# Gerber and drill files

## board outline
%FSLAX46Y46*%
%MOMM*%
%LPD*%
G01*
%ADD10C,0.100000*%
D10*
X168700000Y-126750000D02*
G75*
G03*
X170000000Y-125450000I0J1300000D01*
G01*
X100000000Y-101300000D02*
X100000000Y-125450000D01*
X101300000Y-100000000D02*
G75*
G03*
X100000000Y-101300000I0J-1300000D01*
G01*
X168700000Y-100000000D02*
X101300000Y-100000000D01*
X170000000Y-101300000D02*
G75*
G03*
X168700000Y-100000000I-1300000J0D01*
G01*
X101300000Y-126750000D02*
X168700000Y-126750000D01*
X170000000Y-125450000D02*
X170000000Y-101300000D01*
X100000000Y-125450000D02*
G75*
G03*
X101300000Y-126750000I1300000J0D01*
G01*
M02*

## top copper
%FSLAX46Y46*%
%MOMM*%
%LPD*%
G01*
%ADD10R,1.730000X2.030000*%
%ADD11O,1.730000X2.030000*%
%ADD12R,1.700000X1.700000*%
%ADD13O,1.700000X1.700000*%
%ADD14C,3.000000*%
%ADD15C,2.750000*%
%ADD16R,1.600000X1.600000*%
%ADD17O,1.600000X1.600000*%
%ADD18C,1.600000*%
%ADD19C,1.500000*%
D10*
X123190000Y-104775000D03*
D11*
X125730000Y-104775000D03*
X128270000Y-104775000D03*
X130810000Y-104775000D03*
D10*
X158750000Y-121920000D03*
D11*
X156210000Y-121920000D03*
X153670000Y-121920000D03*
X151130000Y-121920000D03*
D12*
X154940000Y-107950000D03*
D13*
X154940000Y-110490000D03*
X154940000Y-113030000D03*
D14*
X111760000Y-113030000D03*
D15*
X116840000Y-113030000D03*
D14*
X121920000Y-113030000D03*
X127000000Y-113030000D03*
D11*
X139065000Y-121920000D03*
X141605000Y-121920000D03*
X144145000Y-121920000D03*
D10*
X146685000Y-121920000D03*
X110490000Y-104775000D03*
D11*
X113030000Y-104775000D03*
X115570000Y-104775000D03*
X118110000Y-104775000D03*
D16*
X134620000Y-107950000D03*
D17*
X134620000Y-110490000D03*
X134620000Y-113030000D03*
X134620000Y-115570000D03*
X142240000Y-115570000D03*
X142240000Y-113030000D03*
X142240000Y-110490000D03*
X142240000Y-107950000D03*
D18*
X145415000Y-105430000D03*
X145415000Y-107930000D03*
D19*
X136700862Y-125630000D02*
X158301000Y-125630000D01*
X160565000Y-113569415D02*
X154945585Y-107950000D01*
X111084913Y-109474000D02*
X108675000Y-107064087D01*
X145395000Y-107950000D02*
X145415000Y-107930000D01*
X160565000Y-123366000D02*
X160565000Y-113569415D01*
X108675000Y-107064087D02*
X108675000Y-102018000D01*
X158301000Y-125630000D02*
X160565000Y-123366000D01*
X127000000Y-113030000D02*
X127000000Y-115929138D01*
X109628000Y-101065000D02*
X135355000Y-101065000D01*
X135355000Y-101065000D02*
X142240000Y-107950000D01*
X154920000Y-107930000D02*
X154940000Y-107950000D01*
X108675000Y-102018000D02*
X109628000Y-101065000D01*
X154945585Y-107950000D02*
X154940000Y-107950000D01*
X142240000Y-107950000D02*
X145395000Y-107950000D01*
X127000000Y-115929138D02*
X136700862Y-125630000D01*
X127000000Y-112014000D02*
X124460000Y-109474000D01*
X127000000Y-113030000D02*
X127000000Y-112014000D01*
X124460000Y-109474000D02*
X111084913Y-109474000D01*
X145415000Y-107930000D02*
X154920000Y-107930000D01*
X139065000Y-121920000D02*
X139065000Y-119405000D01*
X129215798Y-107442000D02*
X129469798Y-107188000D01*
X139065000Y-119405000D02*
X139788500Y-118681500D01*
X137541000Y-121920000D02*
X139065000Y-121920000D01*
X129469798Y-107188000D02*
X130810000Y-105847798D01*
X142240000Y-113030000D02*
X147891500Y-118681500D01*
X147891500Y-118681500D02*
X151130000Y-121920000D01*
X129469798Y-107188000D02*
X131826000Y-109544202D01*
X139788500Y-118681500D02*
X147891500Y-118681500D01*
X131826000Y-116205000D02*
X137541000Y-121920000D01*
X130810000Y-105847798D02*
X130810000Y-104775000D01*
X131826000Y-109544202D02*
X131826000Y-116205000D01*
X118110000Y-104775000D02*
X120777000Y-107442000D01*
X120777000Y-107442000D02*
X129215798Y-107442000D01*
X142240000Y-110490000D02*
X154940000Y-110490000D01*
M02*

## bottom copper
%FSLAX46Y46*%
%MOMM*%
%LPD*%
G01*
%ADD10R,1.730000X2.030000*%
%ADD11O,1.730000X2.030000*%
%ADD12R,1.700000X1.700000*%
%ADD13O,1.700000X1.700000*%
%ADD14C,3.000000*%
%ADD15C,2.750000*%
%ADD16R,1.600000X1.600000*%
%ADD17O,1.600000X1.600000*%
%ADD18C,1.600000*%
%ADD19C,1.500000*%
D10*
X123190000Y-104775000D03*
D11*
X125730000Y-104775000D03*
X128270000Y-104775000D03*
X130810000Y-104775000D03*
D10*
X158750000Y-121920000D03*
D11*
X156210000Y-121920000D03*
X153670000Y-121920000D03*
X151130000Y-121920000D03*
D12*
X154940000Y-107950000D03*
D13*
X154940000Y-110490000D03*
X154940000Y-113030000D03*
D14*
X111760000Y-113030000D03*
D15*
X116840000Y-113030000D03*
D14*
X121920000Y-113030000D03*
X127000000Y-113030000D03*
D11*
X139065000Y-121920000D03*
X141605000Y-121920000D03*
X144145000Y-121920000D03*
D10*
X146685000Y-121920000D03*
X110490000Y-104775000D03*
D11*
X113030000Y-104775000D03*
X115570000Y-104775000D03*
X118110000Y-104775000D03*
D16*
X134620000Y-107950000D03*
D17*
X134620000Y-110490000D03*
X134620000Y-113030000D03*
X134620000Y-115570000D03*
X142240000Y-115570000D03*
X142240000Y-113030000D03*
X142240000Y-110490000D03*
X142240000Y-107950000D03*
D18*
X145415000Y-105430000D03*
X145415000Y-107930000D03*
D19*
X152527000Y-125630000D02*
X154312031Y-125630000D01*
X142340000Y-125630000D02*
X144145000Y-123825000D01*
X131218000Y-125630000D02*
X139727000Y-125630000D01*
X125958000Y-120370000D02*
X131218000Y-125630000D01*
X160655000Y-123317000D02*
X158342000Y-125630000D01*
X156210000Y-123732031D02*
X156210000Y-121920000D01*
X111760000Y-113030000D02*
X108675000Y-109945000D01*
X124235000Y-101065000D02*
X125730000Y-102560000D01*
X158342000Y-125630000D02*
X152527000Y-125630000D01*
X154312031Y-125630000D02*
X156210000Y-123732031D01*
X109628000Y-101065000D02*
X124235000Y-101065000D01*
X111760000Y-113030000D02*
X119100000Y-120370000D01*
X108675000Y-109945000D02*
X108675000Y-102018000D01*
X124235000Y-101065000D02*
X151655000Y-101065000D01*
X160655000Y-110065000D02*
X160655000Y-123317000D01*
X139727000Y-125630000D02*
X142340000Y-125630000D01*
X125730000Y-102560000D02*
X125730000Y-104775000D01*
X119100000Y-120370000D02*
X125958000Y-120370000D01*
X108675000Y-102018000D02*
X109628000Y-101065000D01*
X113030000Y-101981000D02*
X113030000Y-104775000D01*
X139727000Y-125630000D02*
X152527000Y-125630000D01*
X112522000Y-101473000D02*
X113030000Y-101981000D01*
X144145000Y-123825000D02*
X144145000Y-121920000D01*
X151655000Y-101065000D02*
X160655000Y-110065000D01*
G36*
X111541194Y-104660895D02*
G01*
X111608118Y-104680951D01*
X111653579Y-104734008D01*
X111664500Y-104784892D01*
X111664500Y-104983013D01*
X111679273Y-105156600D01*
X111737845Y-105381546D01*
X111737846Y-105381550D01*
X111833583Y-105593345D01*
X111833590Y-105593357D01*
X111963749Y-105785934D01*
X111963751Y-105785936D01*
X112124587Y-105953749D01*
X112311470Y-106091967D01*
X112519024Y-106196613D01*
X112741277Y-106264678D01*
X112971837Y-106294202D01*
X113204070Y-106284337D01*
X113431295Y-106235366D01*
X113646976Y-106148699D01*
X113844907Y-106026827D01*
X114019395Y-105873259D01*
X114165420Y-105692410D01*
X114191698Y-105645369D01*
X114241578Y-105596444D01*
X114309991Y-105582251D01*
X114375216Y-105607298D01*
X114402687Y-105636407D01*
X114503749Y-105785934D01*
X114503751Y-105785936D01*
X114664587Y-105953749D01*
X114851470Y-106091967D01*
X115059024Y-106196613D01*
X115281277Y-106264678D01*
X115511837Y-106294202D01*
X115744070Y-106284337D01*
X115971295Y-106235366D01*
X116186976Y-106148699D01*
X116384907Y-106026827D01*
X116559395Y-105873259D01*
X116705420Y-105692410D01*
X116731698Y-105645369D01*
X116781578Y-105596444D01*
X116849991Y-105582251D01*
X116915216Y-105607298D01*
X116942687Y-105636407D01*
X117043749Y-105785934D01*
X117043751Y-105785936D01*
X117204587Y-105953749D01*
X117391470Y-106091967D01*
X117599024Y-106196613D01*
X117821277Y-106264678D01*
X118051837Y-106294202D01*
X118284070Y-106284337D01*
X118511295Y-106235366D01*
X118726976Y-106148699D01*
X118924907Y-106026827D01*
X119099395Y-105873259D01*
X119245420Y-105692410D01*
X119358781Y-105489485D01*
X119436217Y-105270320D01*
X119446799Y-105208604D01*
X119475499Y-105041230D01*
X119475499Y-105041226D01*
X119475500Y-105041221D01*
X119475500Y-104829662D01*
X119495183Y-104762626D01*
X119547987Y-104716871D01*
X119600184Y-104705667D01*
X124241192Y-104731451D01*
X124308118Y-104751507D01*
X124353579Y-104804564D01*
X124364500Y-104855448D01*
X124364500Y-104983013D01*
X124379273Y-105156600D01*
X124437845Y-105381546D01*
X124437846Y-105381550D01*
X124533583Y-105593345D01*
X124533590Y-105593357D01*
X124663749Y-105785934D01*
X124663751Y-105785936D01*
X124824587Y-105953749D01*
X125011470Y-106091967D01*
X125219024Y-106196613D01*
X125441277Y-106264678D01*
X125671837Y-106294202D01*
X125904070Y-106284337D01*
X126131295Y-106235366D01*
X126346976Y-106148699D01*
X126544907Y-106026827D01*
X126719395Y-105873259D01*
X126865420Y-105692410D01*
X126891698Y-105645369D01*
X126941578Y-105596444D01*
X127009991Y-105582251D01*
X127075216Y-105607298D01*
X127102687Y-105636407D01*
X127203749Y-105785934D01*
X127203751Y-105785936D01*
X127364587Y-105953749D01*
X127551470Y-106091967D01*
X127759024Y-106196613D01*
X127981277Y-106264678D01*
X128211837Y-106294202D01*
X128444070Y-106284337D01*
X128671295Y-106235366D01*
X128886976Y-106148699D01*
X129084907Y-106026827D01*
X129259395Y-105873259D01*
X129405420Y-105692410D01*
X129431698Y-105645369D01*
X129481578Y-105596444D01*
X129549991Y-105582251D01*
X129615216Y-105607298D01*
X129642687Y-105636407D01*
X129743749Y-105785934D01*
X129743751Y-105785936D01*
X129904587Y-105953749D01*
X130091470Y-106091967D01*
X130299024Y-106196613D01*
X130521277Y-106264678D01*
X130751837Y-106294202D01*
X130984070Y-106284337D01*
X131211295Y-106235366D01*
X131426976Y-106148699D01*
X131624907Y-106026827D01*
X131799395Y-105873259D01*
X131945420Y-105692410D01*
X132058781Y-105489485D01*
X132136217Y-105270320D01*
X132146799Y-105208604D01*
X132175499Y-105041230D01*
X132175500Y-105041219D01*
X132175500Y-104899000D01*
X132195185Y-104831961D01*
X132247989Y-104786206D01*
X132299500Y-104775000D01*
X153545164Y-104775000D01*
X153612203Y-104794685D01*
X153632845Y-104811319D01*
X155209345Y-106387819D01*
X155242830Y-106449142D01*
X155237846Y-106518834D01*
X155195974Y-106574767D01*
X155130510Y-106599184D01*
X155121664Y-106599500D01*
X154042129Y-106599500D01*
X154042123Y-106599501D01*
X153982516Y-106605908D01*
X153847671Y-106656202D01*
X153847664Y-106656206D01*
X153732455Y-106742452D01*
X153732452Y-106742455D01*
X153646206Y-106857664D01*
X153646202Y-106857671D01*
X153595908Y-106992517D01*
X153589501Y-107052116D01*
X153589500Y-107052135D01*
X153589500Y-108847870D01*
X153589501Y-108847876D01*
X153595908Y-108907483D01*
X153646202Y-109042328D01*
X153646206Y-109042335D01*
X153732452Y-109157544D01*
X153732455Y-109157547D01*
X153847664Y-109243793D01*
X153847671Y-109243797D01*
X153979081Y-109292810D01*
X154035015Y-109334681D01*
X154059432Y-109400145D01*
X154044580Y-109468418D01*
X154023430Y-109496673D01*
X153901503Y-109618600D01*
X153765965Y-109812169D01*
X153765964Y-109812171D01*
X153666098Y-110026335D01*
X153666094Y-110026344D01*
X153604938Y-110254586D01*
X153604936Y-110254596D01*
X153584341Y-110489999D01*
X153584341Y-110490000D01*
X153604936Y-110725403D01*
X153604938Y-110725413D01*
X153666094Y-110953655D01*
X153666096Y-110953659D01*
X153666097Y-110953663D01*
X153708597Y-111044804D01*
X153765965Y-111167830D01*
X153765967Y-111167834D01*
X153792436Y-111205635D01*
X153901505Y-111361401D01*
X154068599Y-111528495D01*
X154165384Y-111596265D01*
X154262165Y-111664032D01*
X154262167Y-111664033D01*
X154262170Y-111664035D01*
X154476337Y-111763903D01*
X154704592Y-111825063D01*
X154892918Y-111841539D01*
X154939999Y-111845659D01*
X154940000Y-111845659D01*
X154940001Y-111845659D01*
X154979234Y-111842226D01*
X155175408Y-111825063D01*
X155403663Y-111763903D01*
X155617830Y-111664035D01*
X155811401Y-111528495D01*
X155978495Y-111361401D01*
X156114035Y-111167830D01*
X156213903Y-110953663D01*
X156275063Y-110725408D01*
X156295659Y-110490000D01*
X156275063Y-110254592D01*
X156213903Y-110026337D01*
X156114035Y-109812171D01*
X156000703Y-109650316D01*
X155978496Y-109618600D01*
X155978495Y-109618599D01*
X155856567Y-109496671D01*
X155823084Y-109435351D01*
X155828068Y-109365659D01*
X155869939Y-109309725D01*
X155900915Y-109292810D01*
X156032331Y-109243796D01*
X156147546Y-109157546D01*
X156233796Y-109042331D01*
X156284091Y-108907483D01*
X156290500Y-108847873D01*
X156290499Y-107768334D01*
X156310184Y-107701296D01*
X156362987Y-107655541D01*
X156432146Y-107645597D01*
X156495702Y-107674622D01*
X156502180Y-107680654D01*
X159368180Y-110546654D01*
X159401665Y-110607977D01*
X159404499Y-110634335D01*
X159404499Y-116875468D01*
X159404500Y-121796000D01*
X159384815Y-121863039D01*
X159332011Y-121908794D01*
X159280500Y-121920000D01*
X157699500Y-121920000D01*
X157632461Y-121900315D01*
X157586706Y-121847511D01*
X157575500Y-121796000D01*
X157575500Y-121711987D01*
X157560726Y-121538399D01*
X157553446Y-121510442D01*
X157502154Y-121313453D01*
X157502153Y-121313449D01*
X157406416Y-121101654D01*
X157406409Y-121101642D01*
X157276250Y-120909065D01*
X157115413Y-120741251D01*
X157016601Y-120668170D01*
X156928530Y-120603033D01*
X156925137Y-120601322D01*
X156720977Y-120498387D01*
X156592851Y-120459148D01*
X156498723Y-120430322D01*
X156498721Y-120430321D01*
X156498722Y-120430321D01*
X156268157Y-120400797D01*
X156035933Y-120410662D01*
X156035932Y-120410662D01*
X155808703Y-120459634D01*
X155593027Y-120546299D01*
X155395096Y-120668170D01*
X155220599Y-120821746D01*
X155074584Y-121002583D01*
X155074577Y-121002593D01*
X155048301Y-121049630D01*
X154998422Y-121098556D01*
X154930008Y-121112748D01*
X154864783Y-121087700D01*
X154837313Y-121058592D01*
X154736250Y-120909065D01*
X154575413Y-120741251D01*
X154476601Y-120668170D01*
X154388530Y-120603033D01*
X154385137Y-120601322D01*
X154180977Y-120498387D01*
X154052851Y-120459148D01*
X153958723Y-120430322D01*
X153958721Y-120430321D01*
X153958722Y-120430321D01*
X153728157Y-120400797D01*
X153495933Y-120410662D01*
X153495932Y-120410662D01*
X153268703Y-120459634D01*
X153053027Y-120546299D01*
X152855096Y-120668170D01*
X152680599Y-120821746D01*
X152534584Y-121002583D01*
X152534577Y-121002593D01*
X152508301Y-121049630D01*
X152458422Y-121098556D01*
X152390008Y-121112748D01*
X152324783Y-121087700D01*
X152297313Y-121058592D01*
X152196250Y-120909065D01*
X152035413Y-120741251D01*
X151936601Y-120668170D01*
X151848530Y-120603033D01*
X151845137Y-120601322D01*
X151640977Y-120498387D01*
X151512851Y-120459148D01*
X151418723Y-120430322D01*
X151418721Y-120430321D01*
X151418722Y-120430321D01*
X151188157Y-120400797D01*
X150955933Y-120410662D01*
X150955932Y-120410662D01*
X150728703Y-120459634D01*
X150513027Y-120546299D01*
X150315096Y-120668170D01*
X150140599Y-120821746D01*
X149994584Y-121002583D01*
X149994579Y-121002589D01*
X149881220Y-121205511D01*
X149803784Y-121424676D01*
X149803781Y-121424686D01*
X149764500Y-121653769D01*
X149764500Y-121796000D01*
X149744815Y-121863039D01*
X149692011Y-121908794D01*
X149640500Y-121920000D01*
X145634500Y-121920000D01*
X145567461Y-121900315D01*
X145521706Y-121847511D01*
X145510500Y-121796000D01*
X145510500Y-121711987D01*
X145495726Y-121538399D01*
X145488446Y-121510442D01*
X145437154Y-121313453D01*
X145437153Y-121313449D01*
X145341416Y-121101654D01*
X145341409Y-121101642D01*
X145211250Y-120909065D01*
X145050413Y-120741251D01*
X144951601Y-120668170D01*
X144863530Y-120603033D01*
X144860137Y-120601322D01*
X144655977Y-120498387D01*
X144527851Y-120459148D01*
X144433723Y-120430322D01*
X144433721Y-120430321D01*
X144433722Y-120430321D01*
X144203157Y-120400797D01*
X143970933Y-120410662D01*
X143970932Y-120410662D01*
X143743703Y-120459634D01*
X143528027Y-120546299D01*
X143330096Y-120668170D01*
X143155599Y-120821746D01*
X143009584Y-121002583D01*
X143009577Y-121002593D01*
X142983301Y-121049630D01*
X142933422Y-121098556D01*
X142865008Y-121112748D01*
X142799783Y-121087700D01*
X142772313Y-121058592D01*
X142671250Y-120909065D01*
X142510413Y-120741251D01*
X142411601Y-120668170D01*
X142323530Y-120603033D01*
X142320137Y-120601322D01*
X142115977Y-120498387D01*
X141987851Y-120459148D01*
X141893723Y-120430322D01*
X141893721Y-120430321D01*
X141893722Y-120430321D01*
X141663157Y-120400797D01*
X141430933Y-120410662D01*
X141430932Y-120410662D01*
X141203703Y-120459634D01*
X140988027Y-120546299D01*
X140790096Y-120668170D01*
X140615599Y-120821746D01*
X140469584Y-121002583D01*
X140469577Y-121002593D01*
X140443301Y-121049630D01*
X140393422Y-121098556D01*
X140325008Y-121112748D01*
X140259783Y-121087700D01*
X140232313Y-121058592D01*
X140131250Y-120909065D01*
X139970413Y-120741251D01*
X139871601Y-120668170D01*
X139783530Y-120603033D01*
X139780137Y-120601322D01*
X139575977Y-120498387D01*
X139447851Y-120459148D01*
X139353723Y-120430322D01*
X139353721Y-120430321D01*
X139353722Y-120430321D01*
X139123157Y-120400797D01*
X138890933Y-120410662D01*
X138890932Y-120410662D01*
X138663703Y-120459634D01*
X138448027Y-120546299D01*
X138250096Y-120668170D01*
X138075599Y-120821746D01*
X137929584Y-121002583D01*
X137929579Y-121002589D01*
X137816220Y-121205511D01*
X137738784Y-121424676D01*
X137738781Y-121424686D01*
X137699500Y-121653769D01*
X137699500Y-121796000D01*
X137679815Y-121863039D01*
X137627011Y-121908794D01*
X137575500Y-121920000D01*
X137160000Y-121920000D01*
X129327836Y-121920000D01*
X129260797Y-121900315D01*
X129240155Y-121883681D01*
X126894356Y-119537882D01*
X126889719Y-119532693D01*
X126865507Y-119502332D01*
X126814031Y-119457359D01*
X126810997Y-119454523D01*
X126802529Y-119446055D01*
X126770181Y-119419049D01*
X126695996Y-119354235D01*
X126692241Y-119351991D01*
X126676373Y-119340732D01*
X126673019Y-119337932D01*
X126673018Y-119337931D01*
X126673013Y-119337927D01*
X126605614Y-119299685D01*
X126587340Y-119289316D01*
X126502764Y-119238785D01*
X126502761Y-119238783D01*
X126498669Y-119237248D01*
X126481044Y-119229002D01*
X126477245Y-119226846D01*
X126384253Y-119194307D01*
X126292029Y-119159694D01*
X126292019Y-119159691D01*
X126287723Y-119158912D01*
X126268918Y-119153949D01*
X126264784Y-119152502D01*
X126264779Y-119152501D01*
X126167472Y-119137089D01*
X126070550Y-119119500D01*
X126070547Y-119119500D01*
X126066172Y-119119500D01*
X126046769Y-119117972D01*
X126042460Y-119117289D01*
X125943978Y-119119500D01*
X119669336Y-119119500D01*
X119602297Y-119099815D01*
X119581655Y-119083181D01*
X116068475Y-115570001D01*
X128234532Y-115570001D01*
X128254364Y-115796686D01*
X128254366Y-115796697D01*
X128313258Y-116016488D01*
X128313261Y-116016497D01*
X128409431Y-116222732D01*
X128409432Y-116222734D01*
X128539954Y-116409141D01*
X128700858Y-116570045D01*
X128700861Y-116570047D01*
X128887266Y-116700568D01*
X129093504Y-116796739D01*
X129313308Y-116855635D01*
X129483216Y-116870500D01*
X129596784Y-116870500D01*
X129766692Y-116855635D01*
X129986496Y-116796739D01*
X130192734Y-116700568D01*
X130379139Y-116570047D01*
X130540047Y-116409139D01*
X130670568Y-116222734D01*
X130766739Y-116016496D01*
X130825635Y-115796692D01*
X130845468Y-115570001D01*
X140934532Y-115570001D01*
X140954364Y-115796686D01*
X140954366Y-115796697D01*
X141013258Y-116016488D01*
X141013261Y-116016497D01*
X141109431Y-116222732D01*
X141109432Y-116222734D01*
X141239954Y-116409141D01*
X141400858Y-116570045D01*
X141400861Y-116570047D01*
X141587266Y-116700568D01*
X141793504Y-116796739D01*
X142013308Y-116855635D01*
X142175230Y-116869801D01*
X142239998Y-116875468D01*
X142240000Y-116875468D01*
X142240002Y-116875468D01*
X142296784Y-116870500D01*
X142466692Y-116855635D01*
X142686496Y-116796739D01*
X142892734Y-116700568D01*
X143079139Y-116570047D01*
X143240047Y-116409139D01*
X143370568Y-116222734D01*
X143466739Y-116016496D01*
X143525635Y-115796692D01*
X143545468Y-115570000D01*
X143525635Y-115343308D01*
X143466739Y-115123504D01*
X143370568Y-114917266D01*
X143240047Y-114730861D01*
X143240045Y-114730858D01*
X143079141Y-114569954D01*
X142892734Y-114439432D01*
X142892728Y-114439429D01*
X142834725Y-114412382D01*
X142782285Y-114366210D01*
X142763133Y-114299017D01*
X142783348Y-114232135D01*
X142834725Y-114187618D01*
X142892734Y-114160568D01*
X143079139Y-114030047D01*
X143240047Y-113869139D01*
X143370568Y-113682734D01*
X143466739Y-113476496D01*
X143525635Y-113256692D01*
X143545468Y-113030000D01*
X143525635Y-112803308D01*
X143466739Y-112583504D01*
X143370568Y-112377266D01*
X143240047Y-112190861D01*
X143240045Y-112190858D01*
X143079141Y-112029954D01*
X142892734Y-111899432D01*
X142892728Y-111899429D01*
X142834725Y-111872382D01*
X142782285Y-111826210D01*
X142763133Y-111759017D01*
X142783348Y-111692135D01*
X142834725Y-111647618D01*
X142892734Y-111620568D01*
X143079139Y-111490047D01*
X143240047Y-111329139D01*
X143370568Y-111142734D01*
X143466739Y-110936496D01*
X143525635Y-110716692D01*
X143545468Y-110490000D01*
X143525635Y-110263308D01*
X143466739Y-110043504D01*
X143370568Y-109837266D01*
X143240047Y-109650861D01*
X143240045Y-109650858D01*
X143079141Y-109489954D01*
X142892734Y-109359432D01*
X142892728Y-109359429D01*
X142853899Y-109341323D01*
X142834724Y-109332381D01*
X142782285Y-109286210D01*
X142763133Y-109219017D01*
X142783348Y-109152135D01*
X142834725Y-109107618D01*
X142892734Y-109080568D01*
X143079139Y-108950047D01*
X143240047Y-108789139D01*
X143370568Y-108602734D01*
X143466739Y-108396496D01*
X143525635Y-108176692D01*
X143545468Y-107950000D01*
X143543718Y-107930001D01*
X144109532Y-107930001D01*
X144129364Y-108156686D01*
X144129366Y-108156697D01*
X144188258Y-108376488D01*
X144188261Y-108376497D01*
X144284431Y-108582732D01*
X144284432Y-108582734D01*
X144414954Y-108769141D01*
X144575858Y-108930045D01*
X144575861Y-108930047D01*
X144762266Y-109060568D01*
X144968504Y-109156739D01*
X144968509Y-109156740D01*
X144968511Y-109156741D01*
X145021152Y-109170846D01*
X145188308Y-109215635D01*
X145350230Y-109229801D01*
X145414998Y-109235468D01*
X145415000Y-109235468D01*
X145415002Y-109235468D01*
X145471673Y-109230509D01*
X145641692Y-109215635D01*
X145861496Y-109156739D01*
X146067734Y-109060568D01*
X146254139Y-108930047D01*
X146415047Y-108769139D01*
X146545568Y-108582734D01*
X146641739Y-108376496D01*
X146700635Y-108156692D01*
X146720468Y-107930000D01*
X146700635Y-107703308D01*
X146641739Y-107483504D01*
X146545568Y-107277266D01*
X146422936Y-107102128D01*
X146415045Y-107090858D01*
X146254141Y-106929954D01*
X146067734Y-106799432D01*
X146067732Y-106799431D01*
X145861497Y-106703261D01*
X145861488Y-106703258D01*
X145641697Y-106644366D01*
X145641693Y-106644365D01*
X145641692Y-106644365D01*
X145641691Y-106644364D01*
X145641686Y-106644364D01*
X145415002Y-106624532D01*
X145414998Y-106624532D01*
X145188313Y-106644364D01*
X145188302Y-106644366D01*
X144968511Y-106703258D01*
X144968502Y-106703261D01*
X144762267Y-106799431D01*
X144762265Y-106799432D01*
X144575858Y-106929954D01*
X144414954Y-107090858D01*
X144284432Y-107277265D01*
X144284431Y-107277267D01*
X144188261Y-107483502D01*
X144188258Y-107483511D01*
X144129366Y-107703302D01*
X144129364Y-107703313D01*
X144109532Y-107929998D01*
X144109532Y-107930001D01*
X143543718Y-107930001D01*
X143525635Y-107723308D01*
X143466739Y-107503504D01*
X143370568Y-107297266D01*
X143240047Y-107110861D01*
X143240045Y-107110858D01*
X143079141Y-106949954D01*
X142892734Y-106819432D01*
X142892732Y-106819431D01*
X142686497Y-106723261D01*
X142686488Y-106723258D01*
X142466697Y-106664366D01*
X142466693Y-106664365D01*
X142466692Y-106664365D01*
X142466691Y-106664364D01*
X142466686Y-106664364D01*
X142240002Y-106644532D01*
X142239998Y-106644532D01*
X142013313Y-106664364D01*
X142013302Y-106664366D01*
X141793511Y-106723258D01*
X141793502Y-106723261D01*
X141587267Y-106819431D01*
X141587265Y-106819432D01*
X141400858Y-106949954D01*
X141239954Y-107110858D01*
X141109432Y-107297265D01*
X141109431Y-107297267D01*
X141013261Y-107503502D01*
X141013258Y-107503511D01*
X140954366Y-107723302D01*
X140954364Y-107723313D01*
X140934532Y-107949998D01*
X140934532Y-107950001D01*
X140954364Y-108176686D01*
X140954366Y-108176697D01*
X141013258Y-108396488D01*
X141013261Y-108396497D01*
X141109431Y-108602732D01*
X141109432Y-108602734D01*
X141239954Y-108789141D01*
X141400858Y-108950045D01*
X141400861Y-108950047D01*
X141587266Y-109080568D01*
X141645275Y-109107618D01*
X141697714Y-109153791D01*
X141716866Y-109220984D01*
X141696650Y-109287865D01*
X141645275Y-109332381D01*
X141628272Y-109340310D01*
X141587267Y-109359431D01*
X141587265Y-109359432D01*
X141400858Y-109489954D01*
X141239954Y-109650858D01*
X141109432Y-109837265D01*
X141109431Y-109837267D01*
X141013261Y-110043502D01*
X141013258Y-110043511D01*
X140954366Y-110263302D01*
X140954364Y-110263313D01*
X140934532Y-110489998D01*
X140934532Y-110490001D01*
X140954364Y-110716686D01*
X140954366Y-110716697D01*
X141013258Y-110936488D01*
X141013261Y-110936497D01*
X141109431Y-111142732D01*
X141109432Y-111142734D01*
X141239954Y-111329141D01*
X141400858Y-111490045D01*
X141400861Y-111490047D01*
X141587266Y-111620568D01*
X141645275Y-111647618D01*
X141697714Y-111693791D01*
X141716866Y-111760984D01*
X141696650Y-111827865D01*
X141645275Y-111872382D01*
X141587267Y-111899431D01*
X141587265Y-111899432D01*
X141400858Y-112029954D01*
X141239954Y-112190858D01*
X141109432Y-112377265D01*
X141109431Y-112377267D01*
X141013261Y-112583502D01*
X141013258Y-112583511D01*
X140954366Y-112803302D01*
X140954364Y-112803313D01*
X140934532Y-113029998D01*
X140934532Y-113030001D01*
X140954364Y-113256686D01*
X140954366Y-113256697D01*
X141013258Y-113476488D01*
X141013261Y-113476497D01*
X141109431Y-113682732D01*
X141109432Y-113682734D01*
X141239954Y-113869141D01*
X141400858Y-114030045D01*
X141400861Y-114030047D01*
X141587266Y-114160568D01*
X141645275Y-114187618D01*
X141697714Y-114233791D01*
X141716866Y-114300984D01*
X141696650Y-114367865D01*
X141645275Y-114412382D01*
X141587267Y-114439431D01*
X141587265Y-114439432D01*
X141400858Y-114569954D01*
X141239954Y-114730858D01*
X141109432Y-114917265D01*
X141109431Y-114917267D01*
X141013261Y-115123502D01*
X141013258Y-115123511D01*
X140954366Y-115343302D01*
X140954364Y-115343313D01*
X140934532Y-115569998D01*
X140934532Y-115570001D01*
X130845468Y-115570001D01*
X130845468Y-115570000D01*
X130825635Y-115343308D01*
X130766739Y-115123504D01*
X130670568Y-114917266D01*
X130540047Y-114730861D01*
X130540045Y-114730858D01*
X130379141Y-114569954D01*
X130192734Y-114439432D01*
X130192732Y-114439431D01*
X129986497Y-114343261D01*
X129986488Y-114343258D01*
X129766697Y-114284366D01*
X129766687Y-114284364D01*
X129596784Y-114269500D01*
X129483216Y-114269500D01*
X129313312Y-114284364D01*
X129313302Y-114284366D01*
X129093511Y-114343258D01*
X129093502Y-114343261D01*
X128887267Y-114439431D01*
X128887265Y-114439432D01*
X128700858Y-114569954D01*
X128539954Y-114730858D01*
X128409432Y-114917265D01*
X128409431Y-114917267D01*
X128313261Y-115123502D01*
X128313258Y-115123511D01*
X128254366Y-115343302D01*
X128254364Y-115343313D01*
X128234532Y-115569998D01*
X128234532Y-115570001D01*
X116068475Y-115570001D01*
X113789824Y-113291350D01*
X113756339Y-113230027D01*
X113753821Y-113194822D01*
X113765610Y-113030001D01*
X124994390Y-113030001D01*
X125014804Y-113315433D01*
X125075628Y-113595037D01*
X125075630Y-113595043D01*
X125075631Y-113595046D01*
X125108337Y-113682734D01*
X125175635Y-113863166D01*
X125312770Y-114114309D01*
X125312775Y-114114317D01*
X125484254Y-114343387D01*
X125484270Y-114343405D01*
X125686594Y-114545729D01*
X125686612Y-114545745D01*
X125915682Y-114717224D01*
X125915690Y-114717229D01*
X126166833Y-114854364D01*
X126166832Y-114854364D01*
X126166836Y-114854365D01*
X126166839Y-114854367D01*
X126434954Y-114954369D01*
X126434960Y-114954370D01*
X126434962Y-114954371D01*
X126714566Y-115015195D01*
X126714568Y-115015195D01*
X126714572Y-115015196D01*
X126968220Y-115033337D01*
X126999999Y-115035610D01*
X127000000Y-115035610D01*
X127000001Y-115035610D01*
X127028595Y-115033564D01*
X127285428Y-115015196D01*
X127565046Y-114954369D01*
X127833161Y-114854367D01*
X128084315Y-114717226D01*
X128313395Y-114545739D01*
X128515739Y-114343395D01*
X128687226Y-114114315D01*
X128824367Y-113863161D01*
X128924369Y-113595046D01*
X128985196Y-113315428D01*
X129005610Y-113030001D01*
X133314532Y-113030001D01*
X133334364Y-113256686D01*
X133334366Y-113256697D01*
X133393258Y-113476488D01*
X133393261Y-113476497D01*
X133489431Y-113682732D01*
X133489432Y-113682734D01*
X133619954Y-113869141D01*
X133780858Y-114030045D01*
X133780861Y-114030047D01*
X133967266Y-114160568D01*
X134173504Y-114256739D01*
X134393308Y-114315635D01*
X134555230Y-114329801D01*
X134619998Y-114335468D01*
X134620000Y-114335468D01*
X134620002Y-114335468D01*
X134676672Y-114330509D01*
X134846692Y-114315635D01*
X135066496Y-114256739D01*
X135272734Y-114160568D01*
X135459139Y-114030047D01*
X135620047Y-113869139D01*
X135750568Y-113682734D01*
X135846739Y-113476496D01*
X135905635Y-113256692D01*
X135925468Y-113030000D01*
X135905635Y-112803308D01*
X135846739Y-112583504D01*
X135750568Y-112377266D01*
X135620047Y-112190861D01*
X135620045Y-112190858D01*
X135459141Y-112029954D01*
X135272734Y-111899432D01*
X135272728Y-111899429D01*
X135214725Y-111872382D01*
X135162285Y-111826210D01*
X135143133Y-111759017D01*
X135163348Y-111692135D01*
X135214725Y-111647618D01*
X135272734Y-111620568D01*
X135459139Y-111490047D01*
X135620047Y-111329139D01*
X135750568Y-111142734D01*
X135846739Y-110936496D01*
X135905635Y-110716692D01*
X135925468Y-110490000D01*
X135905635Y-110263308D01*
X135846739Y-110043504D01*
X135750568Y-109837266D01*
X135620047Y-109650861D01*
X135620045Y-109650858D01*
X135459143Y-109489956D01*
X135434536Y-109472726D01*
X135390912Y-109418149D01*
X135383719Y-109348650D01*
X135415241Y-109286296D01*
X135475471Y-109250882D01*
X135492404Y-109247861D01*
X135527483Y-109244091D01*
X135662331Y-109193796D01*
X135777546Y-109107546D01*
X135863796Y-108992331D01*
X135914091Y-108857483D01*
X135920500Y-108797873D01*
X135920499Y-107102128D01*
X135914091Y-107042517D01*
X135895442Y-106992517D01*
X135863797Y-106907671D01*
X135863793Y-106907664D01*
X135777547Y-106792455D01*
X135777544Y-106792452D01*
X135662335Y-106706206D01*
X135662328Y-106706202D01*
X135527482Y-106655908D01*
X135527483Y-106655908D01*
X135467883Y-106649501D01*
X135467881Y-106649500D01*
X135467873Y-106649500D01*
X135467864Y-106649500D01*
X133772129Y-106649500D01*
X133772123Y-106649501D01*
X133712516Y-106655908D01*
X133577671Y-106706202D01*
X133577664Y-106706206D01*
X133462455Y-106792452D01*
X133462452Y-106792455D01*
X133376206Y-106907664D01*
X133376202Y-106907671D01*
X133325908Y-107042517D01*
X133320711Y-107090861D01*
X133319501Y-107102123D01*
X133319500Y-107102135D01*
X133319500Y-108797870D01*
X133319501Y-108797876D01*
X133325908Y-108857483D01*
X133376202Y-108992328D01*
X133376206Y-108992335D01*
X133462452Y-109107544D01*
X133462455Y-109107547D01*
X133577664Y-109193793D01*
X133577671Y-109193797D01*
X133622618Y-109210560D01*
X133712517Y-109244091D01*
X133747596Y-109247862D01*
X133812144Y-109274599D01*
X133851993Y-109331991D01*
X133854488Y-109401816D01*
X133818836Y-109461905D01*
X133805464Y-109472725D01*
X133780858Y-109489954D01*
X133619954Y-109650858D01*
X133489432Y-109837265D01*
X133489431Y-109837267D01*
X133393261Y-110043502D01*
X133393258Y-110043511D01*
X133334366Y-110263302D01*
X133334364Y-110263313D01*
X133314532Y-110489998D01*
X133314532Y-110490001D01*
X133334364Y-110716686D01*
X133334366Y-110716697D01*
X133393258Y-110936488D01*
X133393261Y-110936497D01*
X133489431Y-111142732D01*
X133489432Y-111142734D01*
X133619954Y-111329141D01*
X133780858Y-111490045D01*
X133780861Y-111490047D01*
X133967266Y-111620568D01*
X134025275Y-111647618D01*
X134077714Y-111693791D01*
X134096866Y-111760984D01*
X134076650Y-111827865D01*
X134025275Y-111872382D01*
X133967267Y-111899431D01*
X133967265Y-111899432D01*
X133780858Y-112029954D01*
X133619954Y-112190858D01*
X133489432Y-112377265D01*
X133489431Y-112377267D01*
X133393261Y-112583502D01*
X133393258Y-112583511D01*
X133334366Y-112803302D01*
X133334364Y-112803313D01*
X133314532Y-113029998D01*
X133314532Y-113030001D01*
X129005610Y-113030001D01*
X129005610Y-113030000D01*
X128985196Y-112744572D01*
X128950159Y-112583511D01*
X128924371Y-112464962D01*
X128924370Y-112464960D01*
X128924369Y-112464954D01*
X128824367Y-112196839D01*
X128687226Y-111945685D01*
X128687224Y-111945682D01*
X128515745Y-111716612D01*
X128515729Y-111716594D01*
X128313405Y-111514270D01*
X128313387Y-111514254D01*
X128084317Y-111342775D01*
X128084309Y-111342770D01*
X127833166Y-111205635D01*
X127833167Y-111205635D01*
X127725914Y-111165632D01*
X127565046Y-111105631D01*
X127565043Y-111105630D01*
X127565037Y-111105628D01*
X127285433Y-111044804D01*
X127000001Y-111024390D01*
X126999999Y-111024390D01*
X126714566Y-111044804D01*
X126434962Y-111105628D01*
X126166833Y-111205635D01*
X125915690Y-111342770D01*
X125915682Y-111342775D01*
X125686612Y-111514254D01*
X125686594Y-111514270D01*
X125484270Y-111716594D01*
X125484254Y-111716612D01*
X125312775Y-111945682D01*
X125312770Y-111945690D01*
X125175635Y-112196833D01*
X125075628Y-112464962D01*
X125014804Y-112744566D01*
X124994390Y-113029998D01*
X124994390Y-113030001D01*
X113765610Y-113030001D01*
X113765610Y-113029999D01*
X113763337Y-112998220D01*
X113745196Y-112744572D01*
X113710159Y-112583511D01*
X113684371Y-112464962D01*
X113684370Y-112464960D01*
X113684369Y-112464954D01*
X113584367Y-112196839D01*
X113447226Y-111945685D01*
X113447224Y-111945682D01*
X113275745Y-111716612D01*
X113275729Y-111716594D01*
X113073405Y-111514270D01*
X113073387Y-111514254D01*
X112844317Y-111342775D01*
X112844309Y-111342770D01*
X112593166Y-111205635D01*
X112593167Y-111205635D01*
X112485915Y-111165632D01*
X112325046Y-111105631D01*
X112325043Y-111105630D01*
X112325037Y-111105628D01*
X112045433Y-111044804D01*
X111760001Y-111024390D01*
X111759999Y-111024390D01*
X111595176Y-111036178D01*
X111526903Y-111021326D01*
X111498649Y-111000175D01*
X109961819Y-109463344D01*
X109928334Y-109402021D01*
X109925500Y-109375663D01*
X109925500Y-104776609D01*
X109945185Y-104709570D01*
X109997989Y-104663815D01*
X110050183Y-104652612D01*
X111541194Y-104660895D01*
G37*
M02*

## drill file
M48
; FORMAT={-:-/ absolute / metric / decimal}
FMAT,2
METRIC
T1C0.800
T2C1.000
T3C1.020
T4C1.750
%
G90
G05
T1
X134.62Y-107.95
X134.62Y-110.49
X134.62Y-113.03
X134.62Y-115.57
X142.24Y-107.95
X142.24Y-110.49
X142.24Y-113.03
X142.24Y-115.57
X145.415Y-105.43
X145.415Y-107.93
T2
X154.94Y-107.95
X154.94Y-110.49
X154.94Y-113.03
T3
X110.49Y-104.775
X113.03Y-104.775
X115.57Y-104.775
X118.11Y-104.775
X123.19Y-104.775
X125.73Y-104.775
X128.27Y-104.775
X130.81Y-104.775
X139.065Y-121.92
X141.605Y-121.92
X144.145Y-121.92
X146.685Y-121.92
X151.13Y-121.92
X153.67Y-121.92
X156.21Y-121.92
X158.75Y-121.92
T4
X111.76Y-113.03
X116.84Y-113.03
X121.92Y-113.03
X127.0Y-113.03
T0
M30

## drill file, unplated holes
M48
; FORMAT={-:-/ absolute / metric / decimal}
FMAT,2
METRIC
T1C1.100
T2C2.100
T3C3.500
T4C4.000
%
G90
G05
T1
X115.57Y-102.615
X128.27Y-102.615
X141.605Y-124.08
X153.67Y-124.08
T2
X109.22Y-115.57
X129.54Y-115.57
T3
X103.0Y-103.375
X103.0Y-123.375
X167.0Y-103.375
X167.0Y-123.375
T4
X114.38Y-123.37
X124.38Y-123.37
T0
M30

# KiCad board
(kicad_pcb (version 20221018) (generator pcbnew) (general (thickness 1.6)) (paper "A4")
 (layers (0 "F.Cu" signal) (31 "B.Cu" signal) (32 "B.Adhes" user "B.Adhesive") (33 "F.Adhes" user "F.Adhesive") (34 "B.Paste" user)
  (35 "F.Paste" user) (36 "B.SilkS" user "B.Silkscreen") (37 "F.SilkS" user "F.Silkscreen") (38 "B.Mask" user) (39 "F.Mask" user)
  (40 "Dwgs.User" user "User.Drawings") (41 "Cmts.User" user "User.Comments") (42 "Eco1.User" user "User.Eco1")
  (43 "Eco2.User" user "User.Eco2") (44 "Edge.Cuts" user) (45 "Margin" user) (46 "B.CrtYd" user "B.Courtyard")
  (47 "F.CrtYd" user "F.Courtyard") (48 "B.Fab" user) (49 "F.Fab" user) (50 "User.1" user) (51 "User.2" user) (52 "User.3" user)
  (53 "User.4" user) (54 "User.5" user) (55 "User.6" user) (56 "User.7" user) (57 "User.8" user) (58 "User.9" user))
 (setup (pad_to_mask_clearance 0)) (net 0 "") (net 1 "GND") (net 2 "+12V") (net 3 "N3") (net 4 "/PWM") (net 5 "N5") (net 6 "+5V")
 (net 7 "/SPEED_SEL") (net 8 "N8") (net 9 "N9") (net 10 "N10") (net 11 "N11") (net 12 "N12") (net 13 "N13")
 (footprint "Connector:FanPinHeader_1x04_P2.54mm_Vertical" (layer "F.Cu") (at 123.19 104.775)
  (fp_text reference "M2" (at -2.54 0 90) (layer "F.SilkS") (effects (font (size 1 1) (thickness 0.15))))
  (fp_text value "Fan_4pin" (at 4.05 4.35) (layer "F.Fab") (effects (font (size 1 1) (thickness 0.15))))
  (pad "" np_thru_hole circle (at 5.08 -2.16 90) (size 1.1 1.1) (drill 1.1) (layers "*.Cu" "*.Mask"))
  (pad "1" thru_hole rect (at 0 0 90) (size 2.03 1.73) (drill 1.02) (layers "*.Cu" "*.Mask") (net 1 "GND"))
  (pad "2" thru_hole oval (at 2.54 0 90) (size 2.03 1.73) (drill 1.02) (layers "*.Cu" "*.Mask") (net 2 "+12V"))
  (pad "3" thru_hole oval (at 5.08 0 90) (size 2.03 1.73) (drill 1.02) (layers "*.Cu" "*.Mask") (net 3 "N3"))
  (pad "4" thru_hole oval (at 7.62 0 90) (size 2.03 1.73) (drill 1.02) (layers "*.Cu" "*.Mask") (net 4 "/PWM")))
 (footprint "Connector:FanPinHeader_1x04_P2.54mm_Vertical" (layer "F.Cu") (at 158.75 121.92 180)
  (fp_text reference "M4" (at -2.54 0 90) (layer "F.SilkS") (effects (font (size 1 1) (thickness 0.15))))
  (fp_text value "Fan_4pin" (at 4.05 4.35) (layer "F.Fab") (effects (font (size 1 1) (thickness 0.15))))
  (pad "" np_thru_hole circle (at 5.08 -2.16 270) (size 1.1 1.1) (drill 1.1) (layers "*.Cu" "*.Mask"))
  (pad "1" thru_hole rect (at 0 0 270) (size 2.03 1.73) (drill 1.02) (layers "*.Cu" "*.Mask") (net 1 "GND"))
  (pad "2" thru_hole oval (at 2.54 0 270) (size 2.03 1.73) (drill 1.02) (layers "*.Cu" "*.Mask") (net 2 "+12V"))
  (pad "3" thru_hole oval (at 5.08 0 270) (size 2.03 1.73) (drill 1.02) (layers "*.Cu" "*.Mask") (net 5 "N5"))
  (pad "4" thru_hole oval (at 7.62 0 270) (size 2.03 1.73) (drill 1.02) (layers "*.Cu" "*.Mask") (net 4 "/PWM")))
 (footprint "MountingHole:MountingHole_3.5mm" (layer "F.Cu") (at 103 103.375)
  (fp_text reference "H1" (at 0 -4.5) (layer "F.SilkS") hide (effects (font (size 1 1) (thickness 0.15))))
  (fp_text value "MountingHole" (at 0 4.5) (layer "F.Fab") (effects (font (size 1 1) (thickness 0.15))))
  (pad "" np_thru_hole circle (at 0 0) (size 3.5 3.5) (drill 3.5) (layers "*.Cu" "*.Mask")))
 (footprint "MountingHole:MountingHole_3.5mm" (layer "F.Cu") (at 103 123.375)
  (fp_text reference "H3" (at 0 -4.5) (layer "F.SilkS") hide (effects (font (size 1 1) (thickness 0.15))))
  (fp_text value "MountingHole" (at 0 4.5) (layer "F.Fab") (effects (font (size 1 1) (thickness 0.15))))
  (pad "" np_thru_hole circle (at 0 0) (size 3.5 3.5) (drill 3.5) (layers "*.Cu" "*.Mask")))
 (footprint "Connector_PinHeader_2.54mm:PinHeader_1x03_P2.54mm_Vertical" (layer "F.Cu") (at 154.94 107.95)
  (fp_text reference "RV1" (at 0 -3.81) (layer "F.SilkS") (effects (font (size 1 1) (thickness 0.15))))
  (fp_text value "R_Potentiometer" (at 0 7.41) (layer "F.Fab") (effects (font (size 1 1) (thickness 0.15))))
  (pad "1" thru_hole rect (at 0 0) (size 1.7 1.7) (drill 1) (layers "*.Cu" "*.Mask") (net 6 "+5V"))
  (pad "2" thru_hole oval (at 0 2.54) (size 1.7 1.7) (drill 1) (layers "*.Cu" "*.Mask") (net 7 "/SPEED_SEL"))
  (pad "3" thru_hole oval (at 0 5.08) (size 1.7 1.7) (drill 1) (layers "*.Cu" "*.Mask") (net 1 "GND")))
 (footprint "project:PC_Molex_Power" (layer "F.Cu") (at 119.38 113.03 180)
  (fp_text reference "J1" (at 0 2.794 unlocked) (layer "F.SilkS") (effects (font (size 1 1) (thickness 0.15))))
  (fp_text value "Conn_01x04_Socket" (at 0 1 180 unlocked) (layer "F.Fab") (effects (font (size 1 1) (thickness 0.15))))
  (pad "" np_thru_hole circle (at -10.16 -2.54 180) (size 2.1 2.1) (drill 2.1) (layers "*.Mask"))
  (pad "" np_thru_hole circle (at -5 -10.34 180) (size 4 4) (drill 4) (layers "F&B.Cu" "*.Mask"))
  (pad "" np_thru_hole circle (at 5 -10.34 180) (size 4 4) (drill 4) (layers "F&B.Cu" "*.Mask"))
  (pad "" np_thru_hole circle (at 10.16 -2.54 180) (size 2.1 2.1) (drill 2.1) (layers "*.Mask"))
  (pad "1" thru_hole circle (at 7.62 0 180) (size 3 3) (drill 1.75) (layers "*.Cu" "*.Mask") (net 2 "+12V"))
  (pad "2" thru_hole circle (at 2.54 0 180) (size 2.75 2.75) (drill 1.75) (layers "*.Cu" "*.Mask") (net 1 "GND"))
  (pad "3" thru_hole circle (at -2.54 0 180) (size 3 3) (drill 1.75) (layers "*.Cu" "*.Mask") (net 1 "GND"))
  (pad "4" thru_hole circle (at -7.62 0 180) (size 3 3) (drill 1.75) (layers "*.Cu" "*.Mask") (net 6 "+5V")))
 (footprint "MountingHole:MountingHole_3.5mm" (layer "F.Cu") (at 167 123.375)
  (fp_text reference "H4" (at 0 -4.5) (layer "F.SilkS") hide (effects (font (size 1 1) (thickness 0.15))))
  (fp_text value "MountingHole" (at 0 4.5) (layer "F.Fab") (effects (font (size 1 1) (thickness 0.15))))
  (pad "" np_thru_hole circle (at 0 0) (size 3.5 3.5) (drill 3.5) (layers "*.Cu" "*.Mask")))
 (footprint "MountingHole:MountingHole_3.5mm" (layer "F.Cu") (at 167 103.375)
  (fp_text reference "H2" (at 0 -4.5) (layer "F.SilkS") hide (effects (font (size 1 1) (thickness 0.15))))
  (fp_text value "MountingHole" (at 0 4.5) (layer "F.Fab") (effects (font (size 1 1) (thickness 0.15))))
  (pad "" np_thru_hole circle (at 0 0) (size 3.5 3.5) (drill 3.5) (layers "*.Cu" "*.Mask")))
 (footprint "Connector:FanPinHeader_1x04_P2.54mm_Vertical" (layer "F.Cu") (at 146.685 121.92 180)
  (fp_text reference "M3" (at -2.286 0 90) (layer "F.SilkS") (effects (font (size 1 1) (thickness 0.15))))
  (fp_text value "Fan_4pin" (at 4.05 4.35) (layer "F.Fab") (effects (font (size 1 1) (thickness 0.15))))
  (pad "" np_thru_hole circle (at 5.08 -2.16 270) (size 1.1 1.1) (drill 1.1) (layers "*.Cu" "*.Mask"))
  (pad "1" thru_hole rect (at 0 0 270) (size 2.03 1.73) (drill 1.02) (layers "*.Cu" "*.Mask") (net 1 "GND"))
  (pad "2" thru_hole oval (at 2.54 0 270) (size 2.03 1.73) (drill 1.02) (layers "*.Cu" "*.Mask") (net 2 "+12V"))
  (pad "3" thru_hole oval (at 5.08 0 270) (size 2.03 1.73) (drill 1.02) (layers "*.Cu" "*.Mask") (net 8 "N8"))
  (pad "4" thru_hole oval (at 7.62 0 270) (size 2.03 1.73) (drill 1.02) (layers "*.Cu" "*.Mask") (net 4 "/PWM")))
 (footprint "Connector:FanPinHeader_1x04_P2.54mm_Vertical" (layer "F.Cu") (at 110.49 104.775)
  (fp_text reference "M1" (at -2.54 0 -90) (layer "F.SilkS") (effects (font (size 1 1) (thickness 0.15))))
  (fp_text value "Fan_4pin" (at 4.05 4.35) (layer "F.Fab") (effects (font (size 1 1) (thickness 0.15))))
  (pad "" np_thru_hole circle (at 5.08 -2.16 90) (size 1.1 1.1) (drill 1.1) (layers "*.Cu" "*.Mask"))
  (pad "1" thru_hole rect (at 0 0 90) (size 2.03 1.73) (drill 1.02) (layers "*.Cu" "*.Mask") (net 1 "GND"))
  (pad "2" thru_hole oval (at 2.54 0 90) (size 2.03 1.73) (drill 1.02) (layers "*.Cu" "*.Mask") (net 2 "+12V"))
  (pad "3" thru_hole oval (at 5.08 0 90) (size 2.03 1.73) (drill 1.02) (layers "*.Cu" "*.Mask") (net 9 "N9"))
  (pad "4" thru_hole oval (at 7.62 0 90) (size 2.03 1.73) (drill 1.02) (layers "*.Cu" "*.Mask") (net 4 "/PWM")))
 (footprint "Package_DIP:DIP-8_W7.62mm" (layer "F.Cu") (at 134.62 107.95)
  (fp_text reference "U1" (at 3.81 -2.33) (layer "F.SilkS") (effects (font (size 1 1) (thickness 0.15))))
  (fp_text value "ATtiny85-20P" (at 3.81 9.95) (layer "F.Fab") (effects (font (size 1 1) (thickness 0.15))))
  (pad "1" thru_hole rect (at 0 0) (size 1.6 1.6) (drill 0.8) (layers "*.Cu" "*.Mask") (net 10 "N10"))
  (pad "2" thru_hole oval (at 0 2.54) (size 1.6 1.6) (drill 0.8) (layers "*.Cu" "*.Mask") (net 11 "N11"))
  (pad "3" thru_hole oval (at 0 5.08) (size 1.6 1.6) (drill 0.8) (layers "*.Cu" "*.Mask") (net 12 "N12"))
  (pad "4" thru_hole oval (at 0 7.62) (size 1.6 1.6) (drill 0.8) (layers "*.Cu" "*.Mask") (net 1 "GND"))
  (pad "5" thru_hole oval (at 7.62 7.62) (size 1.6 1.6) (drill 0.8) (layers "*.Cu" "*.Mask") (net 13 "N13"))
  (pad "6" thru_hole oval (at 7.62 5.08) (size 1.6 1.6) (drill 0.8) (layers "*.Cu" "*.Mask") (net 4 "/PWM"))
  (pad "7" thru_hole oval (at 7.62 2.54) (size 1.6 1.6) (drill 0.8) (layers "*.Cu" "*.Mask") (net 7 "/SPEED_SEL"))
  (pad "8" thru_hole oval (at 7.62 0) (size 1.6 1.6) (drill 0.8) (layers "*.Cu" "*.Mask") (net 6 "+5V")))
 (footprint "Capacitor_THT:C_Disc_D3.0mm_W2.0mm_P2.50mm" (layer "F.Cu") (at 145.415 105.43 -90)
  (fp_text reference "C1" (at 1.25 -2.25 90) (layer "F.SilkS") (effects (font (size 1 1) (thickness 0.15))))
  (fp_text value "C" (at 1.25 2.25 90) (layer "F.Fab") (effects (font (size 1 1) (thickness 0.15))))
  (pad "1" thru_hole circle (at 0 0 270) (size 1.6 1.6) (drill 0.8) (layers "*.Cu" "*.Mask") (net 1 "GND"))
  (pad "2" thru_hole circle (at 2.5 0 270) (size 1.6 1.6) (drill 0.8) (layers "*.Cu" "*.Mask") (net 6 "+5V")))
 (gr_arc (start 170 125.45) (mid 169.619239 126.369239) (end 168.7 126.75) (stroke (width 0.1) (type default)) (layer "Edge.Cuts"))
 (gr_line (start 100 101.3) (end 100 125.45) (stroke (width 0.1) (type default)) (layer "Edge.Cuts"))
 (gr_arc (start 100 101.3) (mid 100.380761 100.380761) (end 101.3 100) (stroke (width 0.1) (type default)) (layer "Edge.Cuts"))
 (gr_line (start 168.7 100) (end 101.3 100) (stroke (width 0.1) (type default)) (layer "Edge.Cuts"))
 (gr_arc (start 168.7 100) (mid 169.619239 100.380761) (end 170 101.3) (stroke (width 0.1) (type default)) (layer "Edge.Cuts"))
 (gr_line (start 101.3 126.75) (end 168.7 126.75) (stroke (width 0.1) (type default)) (layer "Edge.Cuts"))
 (gr_line (start 170 125.45) (end 170 101.3) (stroke (width 0.1) (type default)) (layer "Edge.Cuts"))
 (gr_arc (start 101.3 126.75) (mid 100.380761 126.369239) (end 100 125.45) (stroke (width 0.1) (type default)) (layer "Edge.Cuts"))
 (segment (start 136.700862 125.63) (end 158.301 125.63) (width 1.5) (layer "F.Cu") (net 6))
 (segment (start 160.565 113.569415) (end 154.945585 107.95) (width 1.5) (layer "F.Cu") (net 6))
 (segment (start 111.084913 109.474) (end 108.675 107.064087) (width 1.5) (layer "F.Cu") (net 6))
 (segment (start 145.395 107.95) (end 145.415 107.93) (width 1.5) (layer "F.Cu") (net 6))
 (segment (start 160.565 123.366) (end 160.565 113.569415) (width 1.5) (layer "F.Cu") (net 6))
 (segment (start 108.675 107.064087) (end 108.675 102.018) (width 1.5) (layer "F.Cu") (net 6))
 (segment (start 158.301 125.63) (end 160.565 123.366) (width 1.5) (layer "F.Cu") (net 6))
 (segment (start 127 113.03) (end 127 115.929138) (width 1.5) (layer "F.Cu") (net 6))
 (segment (start 109.628 101.065) (end 135.355 101.065) (width 1.5) (layer "F.Cu") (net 6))
 (segment (start 135.355 101.065) (end 142.24 107.95) (width 1.5) (layer "F.Cu") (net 6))
 (segment (start 154.92 107.93) (end 154.94 107.95) (width 1.5) (layer "F.Cu") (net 6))
 (segment (start 108.675 102.018) (end 109.628 101.065) (width 1.5) (layer "F.Cu") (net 6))
 (segment (start 154.945585 107.95) (end 154.94 107.95) (width 1.5) (layer "F.Cu") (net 6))
 (segment (start 142.24 107.95) (end 145.395 107.95) (width 1.5) (layer "F.Cu") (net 6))
 (segment (start 127 115.929138) (end 136.700862 125.63) (width 1.5) (layer "F.Cu") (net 6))
 (segment (start 127 112.014) (end 124.46 109.474) (width 1.5) (layer "F.Cu") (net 6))
 (segment (start 127 113.03) (end 127 112.014) (width 1.5) (layer "F.Cu") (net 6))
 (segment (start 124.46 109.474) (end 111.084913 109.474) (width 1.5) (layer "F.Cu") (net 6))
 (segment (start 145.415 107.93) (end 154.92 107.93) (width 1.5) (layer "F.Cu") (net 6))
 (segment (start 152.527 125.63) (end 154.312031 125.63) (width 1.5) (layer "B.Cu") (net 2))
 (segment (start 142.34 125.63) (end 144.145 123.825) (width 1.5) (layer "B.Cu") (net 2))
 (segment (start 131.218 125.63) (end 139.727 125.63) (width 1.5) (layer "B.Cu") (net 2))
 (segment (start 125.958 120.37) (end 131.218 125.63) (width 1.5) (layer "B.Cu") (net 2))
 (segment (start 160.655 123.317) (end 158.342 125.63) (width 1.5) (layer "B.Cu") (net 2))
 (segment (start 156.21 123.732031) (end 156.21 121.92) (width 1.5) (layer "B.Cu") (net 2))
 (segment (start 111.76 113.03) (end 108.675 109.945) (width 1.5) (layer "B.Cu") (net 2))
 (segment (start 124.235 101.065) (end 125.73 102.56) (width 1.5) (layer "B.Cu") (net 2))
 (segment (start 158.342 125.63) (end 152.527 125.63) (width 1.5) (layer "B.Cu") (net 2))
 (segment (start 154.312031 125.63) (end 156.21 123.732031) (width 1.5) (layer "B.Cu") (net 2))
 (segment (start 109.628 101.065) (end 124.235 101.065) (width 1.5) (layer "B.Cu") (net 2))
 (segment (start 111.76 113.03) (end 119.1 120.37) (width 1.5) (layer "B.Cu") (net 2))
 (segment (start 108.675 109.945) (end 108.675 102.018) (width 1.5) (layer "B.Cu") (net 2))
 (segment (start 124.235 101.065) (end 151.655 101.065) (width 1.5) (layer "B.Cu") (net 2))
 (segment (start 160.655 110.065) (end 160.655 123.317) (width 1.5) (layer "B.Cu") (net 2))
 (segment (start 139.727 125.63) (end 142.34 125.63) (width 1.5) (layer "B.Cu") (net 2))
 (segment (start 125.73 102.56) (end 125.73 104.775) (width 1.5) (layer "B.Cu") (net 2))
 (segment (start 119.1 120.37) (end 125.958 120.37) (width 1.5) (layer "B.Cu") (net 2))
 (segment (start 108.675 102.018) (end 109.628 101.065) (width 1.5) (layer "B.Cu") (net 2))
 (segment (start 113.03 101.981) (end 113.03 104.775) (width 1.5) (layer "B.Cu") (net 2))
 (segment (start 139.727 125.63) (end 152.527 125.63) (width 1.5) (layer "B.Cu") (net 2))
 (segment (start 112.522 101.473) (end 113.03 101.981) (width 1.5) (layer "B.Cu") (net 2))
 (segment (start 144.145 123.825) (end 144.145 121.92) (width 1.5) (layer "B.Cu") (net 2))
 (segment (start 151.655 101.065) (end 160.655 110.065) (width 1.5) (layer "B.Cu") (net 2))
 (segment (start 139.065 121.92) (end 139.065 119.405) (width 1.5) (layer "F.Cu") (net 4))
 (segment (start 129.215798 107.442) (end 129.469798 107.188) (width 1.5) (layer "F.Cu") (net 4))
 (segment (start 139.065 119.405) (end 139.7885 118.6815) (width 1.5) (layer "F.Cu") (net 4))
 (segment (start 137.541 121.92) (end 139.065 121.92) (width 1.5) (layer "F.Cu") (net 4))
 (segment (start 129.469798 107.188) (end 130.81 105.847798) (width 1.5) (layer "F.Cu") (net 4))
 (segment (start 142.24 113.03) (end 147.8915 118.6815) (width 1.5) (layer "F.Cu") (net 4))
 (segment (start 147.8915 118.6815) (end 151.13 121.92) (width 1.5) (layer "F.Cu") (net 4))
 (segment (start 129.469798 107.188) (end 131.826 109.544202) (width 1.5) (layer "F.Cu") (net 4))
 (segment (start 139.7885 118.6815) (end 147.8915 118.6815) (width 1.5) (layer "F.Cu") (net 4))
 (segment (start 131.826 116.205) (end 137.541 121.92) (width 1.5) (layer "F.Cu") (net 4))
 (segment (start 130.81 105.847798) (end 130.81 104.775) (width 1.5) (layer "F.Cu") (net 4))
 (segment (start 131.826 109.544202) (end 131.826 116.205) (width 1.5) (layer "F.Cu") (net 4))
 (segment (start 118.11 104.775) (end 120.777 107.442) (width 1.5) (layer "F.Cu") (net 4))
 (segment (start 120.777 107.442) (end 129.215798 107.442) (width 1.5) (layer "F.Cu") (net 4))
 (segment (start 142.24 110.49) (end 154.94 110.49) (width 1.5) (layer "F.Cu") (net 7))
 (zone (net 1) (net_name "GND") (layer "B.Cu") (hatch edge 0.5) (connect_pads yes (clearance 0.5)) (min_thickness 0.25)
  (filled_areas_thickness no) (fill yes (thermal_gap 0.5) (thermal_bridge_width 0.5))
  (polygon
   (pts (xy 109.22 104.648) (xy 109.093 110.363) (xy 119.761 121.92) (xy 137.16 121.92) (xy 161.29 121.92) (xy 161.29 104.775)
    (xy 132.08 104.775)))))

